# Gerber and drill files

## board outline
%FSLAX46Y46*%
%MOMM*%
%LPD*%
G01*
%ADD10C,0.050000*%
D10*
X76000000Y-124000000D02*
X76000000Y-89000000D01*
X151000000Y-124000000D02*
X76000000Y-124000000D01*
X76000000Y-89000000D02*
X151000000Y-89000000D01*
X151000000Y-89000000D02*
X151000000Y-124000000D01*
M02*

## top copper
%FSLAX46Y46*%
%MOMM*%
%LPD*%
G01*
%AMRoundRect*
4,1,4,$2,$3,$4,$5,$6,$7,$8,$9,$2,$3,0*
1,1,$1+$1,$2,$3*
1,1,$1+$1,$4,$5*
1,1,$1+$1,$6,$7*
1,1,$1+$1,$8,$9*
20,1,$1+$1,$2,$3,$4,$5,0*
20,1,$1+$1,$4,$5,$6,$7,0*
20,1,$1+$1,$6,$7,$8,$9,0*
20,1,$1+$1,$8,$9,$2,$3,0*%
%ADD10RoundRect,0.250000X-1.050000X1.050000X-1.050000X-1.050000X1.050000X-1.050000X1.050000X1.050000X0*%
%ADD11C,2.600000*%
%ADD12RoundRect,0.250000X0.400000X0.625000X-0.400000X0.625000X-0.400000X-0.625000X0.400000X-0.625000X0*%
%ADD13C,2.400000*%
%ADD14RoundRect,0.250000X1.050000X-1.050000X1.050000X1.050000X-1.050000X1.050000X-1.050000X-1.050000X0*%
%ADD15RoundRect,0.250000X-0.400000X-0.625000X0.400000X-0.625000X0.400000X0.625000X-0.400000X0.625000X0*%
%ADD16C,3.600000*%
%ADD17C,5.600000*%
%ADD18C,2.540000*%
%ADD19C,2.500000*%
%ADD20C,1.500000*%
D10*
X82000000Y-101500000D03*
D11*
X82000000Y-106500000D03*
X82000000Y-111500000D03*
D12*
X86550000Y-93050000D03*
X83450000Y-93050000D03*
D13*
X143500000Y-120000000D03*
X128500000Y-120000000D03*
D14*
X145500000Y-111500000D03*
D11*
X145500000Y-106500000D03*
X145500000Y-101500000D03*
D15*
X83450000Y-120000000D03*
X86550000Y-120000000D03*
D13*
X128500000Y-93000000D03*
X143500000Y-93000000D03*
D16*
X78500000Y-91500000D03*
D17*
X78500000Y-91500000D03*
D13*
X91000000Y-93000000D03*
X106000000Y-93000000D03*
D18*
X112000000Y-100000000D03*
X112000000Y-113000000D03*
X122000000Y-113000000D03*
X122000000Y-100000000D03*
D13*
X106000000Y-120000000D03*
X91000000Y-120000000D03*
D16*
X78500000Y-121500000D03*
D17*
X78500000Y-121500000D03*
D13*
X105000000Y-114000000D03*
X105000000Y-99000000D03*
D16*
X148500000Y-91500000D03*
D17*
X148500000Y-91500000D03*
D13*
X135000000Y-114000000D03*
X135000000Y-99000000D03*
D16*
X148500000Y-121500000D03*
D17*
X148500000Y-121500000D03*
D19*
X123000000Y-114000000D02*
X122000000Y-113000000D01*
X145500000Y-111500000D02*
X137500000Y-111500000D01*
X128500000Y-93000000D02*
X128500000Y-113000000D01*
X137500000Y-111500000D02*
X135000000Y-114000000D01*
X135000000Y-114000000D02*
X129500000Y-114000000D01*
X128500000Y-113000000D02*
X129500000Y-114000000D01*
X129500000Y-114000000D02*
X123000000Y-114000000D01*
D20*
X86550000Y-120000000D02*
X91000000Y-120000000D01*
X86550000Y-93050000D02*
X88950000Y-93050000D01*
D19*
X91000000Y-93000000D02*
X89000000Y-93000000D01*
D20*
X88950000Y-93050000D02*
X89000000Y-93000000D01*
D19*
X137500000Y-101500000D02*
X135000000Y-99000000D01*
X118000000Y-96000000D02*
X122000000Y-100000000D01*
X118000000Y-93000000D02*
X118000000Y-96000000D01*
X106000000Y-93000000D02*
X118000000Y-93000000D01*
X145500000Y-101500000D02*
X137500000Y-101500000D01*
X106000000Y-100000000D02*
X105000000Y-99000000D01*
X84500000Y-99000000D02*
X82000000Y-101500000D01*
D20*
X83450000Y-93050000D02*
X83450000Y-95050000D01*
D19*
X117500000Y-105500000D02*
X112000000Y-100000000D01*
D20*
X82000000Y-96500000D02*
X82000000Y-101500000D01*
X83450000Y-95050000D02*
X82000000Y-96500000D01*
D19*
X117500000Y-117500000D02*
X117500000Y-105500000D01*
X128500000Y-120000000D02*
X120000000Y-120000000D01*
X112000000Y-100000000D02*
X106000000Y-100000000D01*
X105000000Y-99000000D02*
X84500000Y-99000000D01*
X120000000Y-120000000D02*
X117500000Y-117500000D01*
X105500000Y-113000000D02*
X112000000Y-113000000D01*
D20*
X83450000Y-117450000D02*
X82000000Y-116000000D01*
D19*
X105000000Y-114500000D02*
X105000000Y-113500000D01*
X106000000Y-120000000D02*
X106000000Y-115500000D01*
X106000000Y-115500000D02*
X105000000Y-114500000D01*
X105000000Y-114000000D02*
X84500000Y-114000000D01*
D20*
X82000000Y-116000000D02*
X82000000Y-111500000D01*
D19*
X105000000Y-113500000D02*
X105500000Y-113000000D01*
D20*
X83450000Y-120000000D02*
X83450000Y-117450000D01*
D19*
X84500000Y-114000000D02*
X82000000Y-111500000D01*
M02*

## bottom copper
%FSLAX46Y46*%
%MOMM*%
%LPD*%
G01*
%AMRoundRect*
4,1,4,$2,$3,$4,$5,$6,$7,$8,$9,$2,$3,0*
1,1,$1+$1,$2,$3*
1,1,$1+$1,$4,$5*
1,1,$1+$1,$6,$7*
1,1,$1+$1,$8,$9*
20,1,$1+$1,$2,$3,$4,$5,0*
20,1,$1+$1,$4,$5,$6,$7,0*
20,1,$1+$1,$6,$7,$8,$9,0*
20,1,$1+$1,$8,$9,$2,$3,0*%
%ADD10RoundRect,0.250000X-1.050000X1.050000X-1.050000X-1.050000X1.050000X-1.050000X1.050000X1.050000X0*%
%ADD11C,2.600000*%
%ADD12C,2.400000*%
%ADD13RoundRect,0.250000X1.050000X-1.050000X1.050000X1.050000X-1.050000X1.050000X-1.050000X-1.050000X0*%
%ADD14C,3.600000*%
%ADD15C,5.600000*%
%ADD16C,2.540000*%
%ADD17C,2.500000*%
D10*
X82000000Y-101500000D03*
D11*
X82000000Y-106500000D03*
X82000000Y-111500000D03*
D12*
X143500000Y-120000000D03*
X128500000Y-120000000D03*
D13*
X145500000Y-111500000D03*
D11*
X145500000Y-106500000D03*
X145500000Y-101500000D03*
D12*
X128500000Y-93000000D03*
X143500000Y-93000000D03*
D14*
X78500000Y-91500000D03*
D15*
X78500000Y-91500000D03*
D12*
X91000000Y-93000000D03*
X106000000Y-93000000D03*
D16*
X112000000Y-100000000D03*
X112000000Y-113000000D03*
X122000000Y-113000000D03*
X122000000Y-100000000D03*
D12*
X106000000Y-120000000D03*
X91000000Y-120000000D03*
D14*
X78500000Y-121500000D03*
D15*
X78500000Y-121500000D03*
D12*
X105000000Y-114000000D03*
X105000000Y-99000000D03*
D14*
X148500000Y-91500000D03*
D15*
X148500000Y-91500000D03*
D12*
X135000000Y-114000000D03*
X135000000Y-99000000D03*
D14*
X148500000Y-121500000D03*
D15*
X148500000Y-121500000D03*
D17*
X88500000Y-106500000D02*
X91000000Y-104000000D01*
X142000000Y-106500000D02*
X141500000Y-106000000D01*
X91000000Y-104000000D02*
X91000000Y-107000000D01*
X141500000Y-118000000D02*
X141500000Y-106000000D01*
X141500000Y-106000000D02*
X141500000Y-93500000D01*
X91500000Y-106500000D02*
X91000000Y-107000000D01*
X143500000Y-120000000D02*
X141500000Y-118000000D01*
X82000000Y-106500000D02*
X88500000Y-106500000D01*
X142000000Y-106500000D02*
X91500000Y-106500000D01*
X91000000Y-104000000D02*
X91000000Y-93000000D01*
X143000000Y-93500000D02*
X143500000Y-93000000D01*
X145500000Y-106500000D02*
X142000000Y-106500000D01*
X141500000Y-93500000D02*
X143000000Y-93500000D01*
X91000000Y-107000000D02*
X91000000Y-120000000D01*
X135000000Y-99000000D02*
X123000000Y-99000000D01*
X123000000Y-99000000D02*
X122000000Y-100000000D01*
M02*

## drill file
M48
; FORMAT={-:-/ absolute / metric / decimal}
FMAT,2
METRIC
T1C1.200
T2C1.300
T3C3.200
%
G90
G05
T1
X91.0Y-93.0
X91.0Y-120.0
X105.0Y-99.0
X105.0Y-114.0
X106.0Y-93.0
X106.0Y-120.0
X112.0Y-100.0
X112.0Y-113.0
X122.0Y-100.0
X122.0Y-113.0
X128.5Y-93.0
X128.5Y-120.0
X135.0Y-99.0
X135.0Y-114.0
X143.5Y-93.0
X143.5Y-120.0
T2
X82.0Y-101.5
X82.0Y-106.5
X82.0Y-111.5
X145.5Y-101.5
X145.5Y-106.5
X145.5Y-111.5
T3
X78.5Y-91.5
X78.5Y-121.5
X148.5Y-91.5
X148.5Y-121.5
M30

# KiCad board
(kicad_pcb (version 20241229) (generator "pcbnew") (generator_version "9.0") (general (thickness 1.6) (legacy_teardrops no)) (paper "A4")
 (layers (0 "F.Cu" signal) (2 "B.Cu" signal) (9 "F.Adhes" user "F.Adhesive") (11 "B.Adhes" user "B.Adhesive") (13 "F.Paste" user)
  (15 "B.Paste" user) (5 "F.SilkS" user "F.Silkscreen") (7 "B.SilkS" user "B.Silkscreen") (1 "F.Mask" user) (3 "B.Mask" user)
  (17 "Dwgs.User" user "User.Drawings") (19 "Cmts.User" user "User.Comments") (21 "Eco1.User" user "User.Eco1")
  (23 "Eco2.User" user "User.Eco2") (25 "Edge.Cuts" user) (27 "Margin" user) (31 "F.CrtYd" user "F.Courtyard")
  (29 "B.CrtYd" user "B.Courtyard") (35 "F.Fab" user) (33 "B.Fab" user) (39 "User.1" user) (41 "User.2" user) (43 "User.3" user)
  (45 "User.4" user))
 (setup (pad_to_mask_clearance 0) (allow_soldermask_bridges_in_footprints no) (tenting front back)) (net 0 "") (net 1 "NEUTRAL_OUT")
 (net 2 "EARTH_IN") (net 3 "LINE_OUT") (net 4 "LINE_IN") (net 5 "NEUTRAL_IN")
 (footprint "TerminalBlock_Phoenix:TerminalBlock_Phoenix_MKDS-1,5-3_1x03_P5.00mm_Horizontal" (layer "F.Cu") (at 82 101.5 -90)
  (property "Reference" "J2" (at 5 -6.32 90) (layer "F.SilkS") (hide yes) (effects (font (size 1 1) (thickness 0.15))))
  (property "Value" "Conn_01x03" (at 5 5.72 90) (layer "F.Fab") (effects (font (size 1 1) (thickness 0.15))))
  (pad "1" thru_hole roundrect (at 0 0 270) (size 2.6 2.6) (drill 1.3) (layers "*.Cu" "*.Mask") (remove_unused_layers no)
   (roundrect_rratio 0.096154) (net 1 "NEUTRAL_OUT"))
  (pad "2" thru_hole circle (at 5 0 270) (size 2.6 2.6) (drill 1.3) (layers "*.Cu" "*.Mask") (remove_unused_layers no) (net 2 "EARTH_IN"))
  (pad "3" thru_hole circle (at 10 0 270) (size 2.6 2.6) (drill 1.3) (layers "*.Cu" "*.Mask") (remove_unused_layers no) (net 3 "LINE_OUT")))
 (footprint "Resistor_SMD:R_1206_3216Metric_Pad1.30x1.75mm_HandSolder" (layer "F.Cu") (at 85 93.05 180)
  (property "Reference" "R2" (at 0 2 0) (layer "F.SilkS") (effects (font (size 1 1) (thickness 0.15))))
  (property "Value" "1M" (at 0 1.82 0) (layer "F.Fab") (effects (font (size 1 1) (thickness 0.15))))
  (pad "1" smd roundrect (at -1.55 0 180) (size 1.3 1.75) (layers "F.Cu" "F.Mask" "F.Paste") (roundrect_rratio 0.192308) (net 2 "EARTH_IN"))
  (pad "2" smd roundrect (at 1.55 0 180) (size 1.3 1.75) (layers "F.Cu" "F.Mask" "F.Paste") (roundrect_rratio 0.192308)
   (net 1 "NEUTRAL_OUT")))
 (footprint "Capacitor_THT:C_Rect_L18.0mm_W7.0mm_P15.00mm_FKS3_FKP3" (layer "F.Cu") (at 143.5 120 180)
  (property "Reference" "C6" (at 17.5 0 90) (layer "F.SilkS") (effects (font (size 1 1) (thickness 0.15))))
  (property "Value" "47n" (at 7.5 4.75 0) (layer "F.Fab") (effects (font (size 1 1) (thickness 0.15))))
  (pad "1" thru_hole circle (at 0 0 180) (size 2.4 2.4) (drill 1.2) (layers "*.Cu" "*.Mask") (remove_unused_layers no) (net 2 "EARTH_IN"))
  (pad "2" thru_hole circle (at 15 0 180) (size 2.4 2.4) (drill 1.2) (layers "*.Cu" "*.Mask") (remove_unused_layers no)
   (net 1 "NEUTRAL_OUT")))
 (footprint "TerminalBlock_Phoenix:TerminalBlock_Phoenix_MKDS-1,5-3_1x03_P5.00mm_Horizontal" (layer "F.Cu") (at 145.5 111.5 90)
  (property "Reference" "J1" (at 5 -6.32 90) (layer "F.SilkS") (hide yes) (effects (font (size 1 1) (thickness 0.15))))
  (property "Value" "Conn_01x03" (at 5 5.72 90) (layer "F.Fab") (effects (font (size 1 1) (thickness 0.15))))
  (pad "1" thru_hole roundrect (at 0 0 90) (size 2.6 2.6) (drill 1.3) (layers "*.Cu" "*.Mask") (remove_unused_layers no)
   (roundrect_rratio 0.096154) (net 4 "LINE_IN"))
  (pad "2" thru_hole circle (at 5 0 90) (size 2.6 2.6) (drill 1.3) (layers "*.Cu" "*.Mask") (remove_unused_layers no) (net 2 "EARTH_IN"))
  (pad "3" thru_hole circle (at 10 0 90) (size 2.6 2.6) (drill 1.3) (layers "*.Cu" "*.Mask") (remove_unused_layers no) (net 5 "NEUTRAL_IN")))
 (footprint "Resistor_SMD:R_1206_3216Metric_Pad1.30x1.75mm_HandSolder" (layer "F.Cu") (at 85 120)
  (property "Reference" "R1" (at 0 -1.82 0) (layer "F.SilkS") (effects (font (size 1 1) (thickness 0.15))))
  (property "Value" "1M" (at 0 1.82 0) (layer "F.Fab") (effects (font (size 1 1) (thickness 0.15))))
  (pad "1" smd roundrect (at -1.55 0) (size 1.3 1.75) (layers "F.Cu" "F.Mask" "F.Paste") (roundrect_rratio 0.192308) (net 3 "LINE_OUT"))
  (pad "2" smd roundrect (at 1.55 0) (size 1.3 1.75) (layers "F.Cu" "F.Mask" "F.Paste") (roundrect_rratio 0.192308) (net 2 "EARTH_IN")))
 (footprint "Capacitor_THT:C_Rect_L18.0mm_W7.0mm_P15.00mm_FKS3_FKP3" (layer "F.Cu") (at 128.5 93)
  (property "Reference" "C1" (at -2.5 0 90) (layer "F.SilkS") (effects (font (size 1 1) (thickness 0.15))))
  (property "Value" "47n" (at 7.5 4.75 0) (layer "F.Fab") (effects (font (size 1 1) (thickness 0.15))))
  (pad "1" thru_hole circle (at 0 0) (size 2.4 2.4) (drill 1.2) (layers "*.Cu" "*.Mask") (remove_unused_layers no) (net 4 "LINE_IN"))
  (pad "2" thru_hole circle (at 15 0) (size 2.4 2.4) (drill 1.2) (layers "*.Cu" "*.Mask") (remove_unused_layers no) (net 2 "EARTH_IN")))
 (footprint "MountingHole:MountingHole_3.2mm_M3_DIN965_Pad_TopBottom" (layer "F.Cu") (at 78.5 91.5 90)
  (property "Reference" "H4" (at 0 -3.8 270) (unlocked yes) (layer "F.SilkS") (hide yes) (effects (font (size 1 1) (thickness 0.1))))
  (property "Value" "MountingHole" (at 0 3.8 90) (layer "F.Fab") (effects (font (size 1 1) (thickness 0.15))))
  (pad "1" thru_hole circle (at 0 0 90) (size 3.6 3.6) (drill 3.2) (layers "*.Cu" "*.Mask") (remove_unused_layers no))
  (pad "1" connect circle (at 0 0 90) (size 5.6 5.6) (layers "F.Cu" "F.Mask"))
  (pad "1" connect circle (at 0 0 90) (size 5.6 5.6) (layers "B.Cu" "B.Mask")))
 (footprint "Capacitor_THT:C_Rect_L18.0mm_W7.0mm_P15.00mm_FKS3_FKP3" (layer "F.Cu") (at 91 93)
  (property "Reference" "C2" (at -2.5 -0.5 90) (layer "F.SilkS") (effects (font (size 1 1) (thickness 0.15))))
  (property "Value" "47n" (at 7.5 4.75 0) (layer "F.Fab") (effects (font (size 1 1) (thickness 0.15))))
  (pad "1" thru_hole circle (at 0 0) (size 2.4 2.4) (drill 1.2) (layers "*.Cu" "*.Mask") (remove_unused_layers no) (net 2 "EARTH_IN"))
  (pad "2" thru_hole circle (at 15 0) (size 2.4 2.4) (drill 1.2) (layers "*.Cu" "*.Mask") (remove_unused_layers no) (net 5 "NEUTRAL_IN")))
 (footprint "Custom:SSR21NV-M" (layer "F.Cu") (at 117 106.5 -90)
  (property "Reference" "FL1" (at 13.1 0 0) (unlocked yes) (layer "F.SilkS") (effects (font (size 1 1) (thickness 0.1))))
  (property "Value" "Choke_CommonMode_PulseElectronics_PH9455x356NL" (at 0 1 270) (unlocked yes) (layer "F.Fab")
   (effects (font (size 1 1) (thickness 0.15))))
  (pad "1" thru_hole circle (at -6.5 5 270) (size 2.54 2.54) (drill 1.2) (layers "*.Cu" "*.Mask") (remove_unused_layers no)
   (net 1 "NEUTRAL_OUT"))
  (pad "2" thru_hole circle (at 6.5 5 270) (size 2.54 2.54) (drill 1.2) (layers "*.Cu" "*.Mask") (remove_unused_layers no)
   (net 3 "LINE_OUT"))
  (pad "3" thru_hole circle (at 6.5 -5 270) (size 2.54 2.54) (drill 1.2) (layers "*.Cu" "*.Mask") (remove_unused_layers no)
   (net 4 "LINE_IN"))
  (pad "4" thru_hole circle (at -6.5 -5 270) (size 2.54 2.54) (drill 1.2) (layers "*.Cu" "*.Mask") (remove_unused_layers no)
   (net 5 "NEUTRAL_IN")))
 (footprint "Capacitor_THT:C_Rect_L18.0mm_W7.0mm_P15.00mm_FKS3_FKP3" (layer "F.Cu") (at 106 120 180)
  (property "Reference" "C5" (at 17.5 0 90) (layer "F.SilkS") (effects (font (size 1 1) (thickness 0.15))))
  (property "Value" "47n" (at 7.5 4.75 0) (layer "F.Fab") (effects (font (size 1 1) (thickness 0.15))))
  (pad "1" thru_hole circle (at 0 0 180) (size 2.4 2.4) (drill 1.2) (layers "*.Cu" "*.Mask") (remove_unused_layers no) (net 3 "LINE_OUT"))
  (pad "2" thru_hole circle (at 15 0 180) (size 2.4 2.4) (drill 1.2) (layers "*.Cu" "*.Mask") (remove_unused_layers no) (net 2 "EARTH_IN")))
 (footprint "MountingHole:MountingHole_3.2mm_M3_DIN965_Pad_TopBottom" (layer "F.Cu") (at 78.5 121.5 90)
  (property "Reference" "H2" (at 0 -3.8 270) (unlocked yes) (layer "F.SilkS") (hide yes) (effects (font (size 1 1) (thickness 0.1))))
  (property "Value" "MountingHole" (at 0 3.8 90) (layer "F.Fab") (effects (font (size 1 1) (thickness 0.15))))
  (pad "1" thru_hole circle (at 0 0 90) (size 3.6 3.6) (drill 3.2) (layers "*.Cu" "*.Mask") (remove_unused_layers no))
  (pad "1" connect circle (at 0 0 90) (size 5.6 5.6) (layers "F.Cu" "F.Mask"))
  (pad "1" connect circle (at 0 0 90) (size 5.6 5.6) (layers "B.Cu" "B.Mask")))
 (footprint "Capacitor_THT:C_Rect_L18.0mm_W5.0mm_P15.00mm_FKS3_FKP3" (layer "F.Cu") (at 105 114 90)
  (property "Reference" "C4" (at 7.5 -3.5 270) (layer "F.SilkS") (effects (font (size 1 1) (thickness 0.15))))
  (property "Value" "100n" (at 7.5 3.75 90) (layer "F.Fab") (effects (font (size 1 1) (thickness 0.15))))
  (pad "1" thru_hole circle (at 0 0 90) (size 2.4 2.4) (drill 1.2) (layers "*.Cu" "*.Mask") (remove_unused_layers no) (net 3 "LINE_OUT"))
  (pad "2" thru_hole circle (at 15 0 90) (size 2.4 2.4) (drill 1.2) (layers "*.Cu" "*.Mask") (remove_unused_layers no) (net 1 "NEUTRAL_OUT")))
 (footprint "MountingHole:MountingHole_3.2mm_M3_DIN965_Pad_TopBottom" (layer "F.Cu") (at 148.5 91.5 90)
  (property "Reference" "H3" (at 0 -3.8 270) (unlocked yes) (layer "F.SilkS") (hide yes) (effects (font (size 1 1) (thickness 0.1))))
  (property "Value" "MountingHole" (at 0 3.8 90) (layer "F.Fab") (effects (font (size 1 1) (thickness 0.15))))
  (pad "1" thru_hole circle (at 0 0 90) (size 3.6 3.6) (drill 3.2) (layers "*.Cu" "*.Mask") (remove_unused_layers no))
  (pad "1" connect circle (at 0 0 90) (size 5.6 5.6) (layers "F.Cu" "F.Mask"))
  (pad "1" connect circle (at 0 0 90) (size 5.6 5.6) (layers "B.Cu" "B.Mask")))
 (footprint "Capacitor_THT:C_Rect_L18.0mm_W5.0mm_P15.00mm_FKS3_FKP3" (layer "F.Cu") (at 135 114 90)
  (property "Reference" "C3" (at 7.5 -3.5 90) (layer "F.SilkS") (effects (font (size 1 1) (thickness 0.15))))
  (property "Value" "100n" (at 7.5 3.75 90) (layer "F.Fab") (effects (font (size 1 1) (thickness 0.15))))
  (pad "1" thru_hole circle (at 0 0 90) (size 2.4 2.4) (drill 1.2) (layers "*.Cu" "*.Mask") (remove_unused_layers no) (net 4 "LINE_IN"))
  (pad "2" thru_hole circle (at 15 0 90) (size 2.4 2.4) (drill 1.2) (layers "*.Cu" "*.Mask") (remove_unused_layers no) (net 5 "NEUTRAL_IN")))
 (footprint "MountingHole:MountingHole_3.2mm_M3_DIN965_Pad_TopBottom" (layer "F.Cu") (at 148.5 121.5 90)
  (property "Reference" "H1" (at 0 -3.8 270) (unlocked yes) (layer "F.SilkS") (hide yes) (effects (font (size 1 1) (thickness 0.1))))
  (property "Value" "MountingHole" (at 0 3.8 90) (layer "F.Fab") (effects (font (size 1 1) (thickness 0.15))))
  (pad "1" thru_hole circle (at 0 0 90) (size 3.6 3.6) (drill 3.2) (layers "*.Cu" "*.Mask") (remove_unused_layers no))
  (pad "1" connect circle (at 0 0 90) (size 5.6 5.6) (layers "F.Cu" "F.Mask"))
  (pad "1" connect circle (at 0 0 90) (size 5.6 5.6) (layers "B.Cu" "B.Mask")))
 (gr_line (start 76 124) (end 76 89) (stroke (width 0.05) (type default)) (layer "Edge.Cuts"))
 (gr_line (start 151 124) (end 76 124) (stroke (width 0.05) (type default)) (layer "Edge.Cuts"))
 (gr_line (start 76 89) (end 151 89) (stroke (width 0.05) (type default)) (layer "Edge.Cuts"))
 (gr_line (start 151 89) (end 151 124) (stroke (width 0.05) (type default)) (layer "Edge.Cuts"))
 (segment (start 123 114) (end 122 113) (width 2.5) (layer "F.Cu") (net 4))
 (segment (start 145.5 111.5) (end 137.5 111.5) (width 2.5) (layer "F.Cu") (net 4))
 (segment (start 128.5 93) (end 128.5 113) (width 2.5) (layer "F.Cu") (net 4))
 (segment (start 137.5 111.5) (end 135 114) (width 2.5) (layer "F.Cu") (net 4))
 (segment (start 135 114) (end 129.5 114) (width 2.5) (layer "F.Cu") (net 4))
 (segment (start 128.5 113) (end 129.5 114) (width 2.5) (layer "F.Cu") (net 4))
 (segment (start 129.5 114) (end 123 114) (width 2.5) (layer "F.Cu") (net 4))
 (segment (start 86.55 120) (end 91 120) (width 1.5) (layer "F.Cu") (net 2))
 (segment (start 86.55 93.05) (end 88.95 93.05) (width 1.5) (layer "F.Cu") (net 2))
 (segment (start 91 93) (end 89 93) (width 2.5) (layer "F.Cu") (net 2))
 (segment (start 88.95 93.05) (end 89 93) (width 1.5) (layer "F.Cu") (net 2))
 (segment (start 88.5 106.5) (end 91 104) (width 2.5) (layer "B.Cu") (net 2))
 (segment (start 142 106.5) (end 141.5 106) (width 2.5) (layer "B.Cu") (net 2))
 (segment (start 91 104) (end 91 107) (width 2.5) (layer "B.Cu") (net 2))
 (segment (start 141.5 118) (end 141.5 106) (width 2.5) (layer "B.Cu") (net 2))
 (segment (start 141.5 106) (end 141.5 93.5) (width 2.5) (layer "B.Cu") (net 2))
 (segment (start 91.5 106.5) (end 91 107) (width 2.5) (layer "B.Cu") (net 2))
 (segment (start 143.5 120) (end 141.5 118) (width 2.5) (layer "B.Cu") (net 2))
 (segment (start 82 106.5) (end 88.5 106.5) (width 2.5) (layer "B.Cu") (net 2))
 (segment (start 142 106.5) (end 91.5 106.5) (width 2.5) (layer "B.Cu") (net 2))
 (segment (start 91 104) (end 91 93) (width 2.5) (layer "B.Cu") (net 2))
 (segment (start 143 93.5) (end 143.5 93) (width 2.5) (layer "B.Cu") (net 2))
 (segment (start 145.5 106.5) (end 142 106.5) (width 2.5) (layer "B.Cu") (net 2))
 (segment (start 141.5 93.5) (end 143 93.5) (width 2.5) (layer "B.Cu") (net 2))
 (segment (start 91 107) (end 91 120) (width 2.5) (layer "B.Cu") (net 2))
 (segment (start 137.5 101.5) (end 135 99) (width 2.5) (layer "F.Cu") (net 5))
 (segment (start 118 96) (end 122 100) (width 2.5) (layer "F.Cu") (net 5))
 (segment (start 118 93) (end 118 96) (width 2.5) (layer "F.Cu") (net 5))
 (segment (start 106 93) (end 118 93) (width 2.5) (layer "F.Cu") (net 5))
 (segment (start 145.5 101.5) (end 137.5 101.5) (width 2.5) (layer "F.Cu") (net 5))
 (segment (start 135 99) (end 123 99) (width 2.5) (layer "B.Cu") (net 5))
 (segment (start 123 99) (end 122 100) (width 2.5) (layer "B.Cu") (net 5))
 (segment (start 106 100) (end 105 99) (width 2.5) (layer "F.Cu") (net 1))
 (segment (start 84.5 99) (end 82 101.5) (width 2.5) (layer "F.Cu") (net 1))
 (segment (start 83.45 93.05) (end 83.45 95.05) (width 1.5) (layer "F.Cu") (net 1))
 (segment (start 117.5 105.5) (end 112 100) (width 2.5) (layer "F.Cu") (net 1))
 (segment (start 82 96.5) (end 82 101.5) (width 1.5) (layer "F.Cu") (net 1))
 (segment (start 83.45 95.05) (end 82 96.5) (width 1.5) (layer "F.Cu") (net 1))
 (segment (start 117.5 117.5) (end 117.5 105.5) (width 2.5) (layer "F.Cu") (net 1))
 (segment (start 128.5 120) (end 120 120) (width 2.5) (layer "F.Cu") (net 1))
 (segment (start 112 100) (end 106 100) (width 2.5) (layer "F.Cu") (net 1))
 (segment (start 105 99) (end 84.5 99) (width 2.5) (layer "F.Cu") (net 1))
 (segment (start 120 120) (end 117.5 117.5) (width 2.5) (layer "F.Cu") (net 1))
 (segment (start 105.5 113) (end 112 113) (width 2.5) (layer "F.Cu") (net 3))
 (segment (start 83.45 117.45) (end 82 116) (width 1.5) (layer "F.Cu") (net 3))
 (segment (start 105 114.5) (end 105 113.5) (width 2.5) (layer "F.Cu") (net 3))
 (segment (start 106 120) (end 106 115.5) (width 2.5) (layer "F.Cu") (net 3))
 (segment (start 106 115.5) (end 105 114.5) (width 2.5) (layer "F.Cu") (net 3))
 (segment (start 105 114) (end 84.5 114) (width 2.5) (layer "F.Cu") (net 3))
 (segment (start 82 116) (end 82 111.5) (width 1.5) (layer "F.Cu") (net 3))
 (segment (start 105 113.5) (end 105.5 113) (width 2.5) (layer "F.Cu") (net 3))
 (segment (start 83.45 120) (end 83.45 117.45) (width 1.5) (layer "F.Cu") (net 3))
 (segment (start 84.5 114) (end 82 111.5) (width 2.5) (layer "F.Cu") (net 3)))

